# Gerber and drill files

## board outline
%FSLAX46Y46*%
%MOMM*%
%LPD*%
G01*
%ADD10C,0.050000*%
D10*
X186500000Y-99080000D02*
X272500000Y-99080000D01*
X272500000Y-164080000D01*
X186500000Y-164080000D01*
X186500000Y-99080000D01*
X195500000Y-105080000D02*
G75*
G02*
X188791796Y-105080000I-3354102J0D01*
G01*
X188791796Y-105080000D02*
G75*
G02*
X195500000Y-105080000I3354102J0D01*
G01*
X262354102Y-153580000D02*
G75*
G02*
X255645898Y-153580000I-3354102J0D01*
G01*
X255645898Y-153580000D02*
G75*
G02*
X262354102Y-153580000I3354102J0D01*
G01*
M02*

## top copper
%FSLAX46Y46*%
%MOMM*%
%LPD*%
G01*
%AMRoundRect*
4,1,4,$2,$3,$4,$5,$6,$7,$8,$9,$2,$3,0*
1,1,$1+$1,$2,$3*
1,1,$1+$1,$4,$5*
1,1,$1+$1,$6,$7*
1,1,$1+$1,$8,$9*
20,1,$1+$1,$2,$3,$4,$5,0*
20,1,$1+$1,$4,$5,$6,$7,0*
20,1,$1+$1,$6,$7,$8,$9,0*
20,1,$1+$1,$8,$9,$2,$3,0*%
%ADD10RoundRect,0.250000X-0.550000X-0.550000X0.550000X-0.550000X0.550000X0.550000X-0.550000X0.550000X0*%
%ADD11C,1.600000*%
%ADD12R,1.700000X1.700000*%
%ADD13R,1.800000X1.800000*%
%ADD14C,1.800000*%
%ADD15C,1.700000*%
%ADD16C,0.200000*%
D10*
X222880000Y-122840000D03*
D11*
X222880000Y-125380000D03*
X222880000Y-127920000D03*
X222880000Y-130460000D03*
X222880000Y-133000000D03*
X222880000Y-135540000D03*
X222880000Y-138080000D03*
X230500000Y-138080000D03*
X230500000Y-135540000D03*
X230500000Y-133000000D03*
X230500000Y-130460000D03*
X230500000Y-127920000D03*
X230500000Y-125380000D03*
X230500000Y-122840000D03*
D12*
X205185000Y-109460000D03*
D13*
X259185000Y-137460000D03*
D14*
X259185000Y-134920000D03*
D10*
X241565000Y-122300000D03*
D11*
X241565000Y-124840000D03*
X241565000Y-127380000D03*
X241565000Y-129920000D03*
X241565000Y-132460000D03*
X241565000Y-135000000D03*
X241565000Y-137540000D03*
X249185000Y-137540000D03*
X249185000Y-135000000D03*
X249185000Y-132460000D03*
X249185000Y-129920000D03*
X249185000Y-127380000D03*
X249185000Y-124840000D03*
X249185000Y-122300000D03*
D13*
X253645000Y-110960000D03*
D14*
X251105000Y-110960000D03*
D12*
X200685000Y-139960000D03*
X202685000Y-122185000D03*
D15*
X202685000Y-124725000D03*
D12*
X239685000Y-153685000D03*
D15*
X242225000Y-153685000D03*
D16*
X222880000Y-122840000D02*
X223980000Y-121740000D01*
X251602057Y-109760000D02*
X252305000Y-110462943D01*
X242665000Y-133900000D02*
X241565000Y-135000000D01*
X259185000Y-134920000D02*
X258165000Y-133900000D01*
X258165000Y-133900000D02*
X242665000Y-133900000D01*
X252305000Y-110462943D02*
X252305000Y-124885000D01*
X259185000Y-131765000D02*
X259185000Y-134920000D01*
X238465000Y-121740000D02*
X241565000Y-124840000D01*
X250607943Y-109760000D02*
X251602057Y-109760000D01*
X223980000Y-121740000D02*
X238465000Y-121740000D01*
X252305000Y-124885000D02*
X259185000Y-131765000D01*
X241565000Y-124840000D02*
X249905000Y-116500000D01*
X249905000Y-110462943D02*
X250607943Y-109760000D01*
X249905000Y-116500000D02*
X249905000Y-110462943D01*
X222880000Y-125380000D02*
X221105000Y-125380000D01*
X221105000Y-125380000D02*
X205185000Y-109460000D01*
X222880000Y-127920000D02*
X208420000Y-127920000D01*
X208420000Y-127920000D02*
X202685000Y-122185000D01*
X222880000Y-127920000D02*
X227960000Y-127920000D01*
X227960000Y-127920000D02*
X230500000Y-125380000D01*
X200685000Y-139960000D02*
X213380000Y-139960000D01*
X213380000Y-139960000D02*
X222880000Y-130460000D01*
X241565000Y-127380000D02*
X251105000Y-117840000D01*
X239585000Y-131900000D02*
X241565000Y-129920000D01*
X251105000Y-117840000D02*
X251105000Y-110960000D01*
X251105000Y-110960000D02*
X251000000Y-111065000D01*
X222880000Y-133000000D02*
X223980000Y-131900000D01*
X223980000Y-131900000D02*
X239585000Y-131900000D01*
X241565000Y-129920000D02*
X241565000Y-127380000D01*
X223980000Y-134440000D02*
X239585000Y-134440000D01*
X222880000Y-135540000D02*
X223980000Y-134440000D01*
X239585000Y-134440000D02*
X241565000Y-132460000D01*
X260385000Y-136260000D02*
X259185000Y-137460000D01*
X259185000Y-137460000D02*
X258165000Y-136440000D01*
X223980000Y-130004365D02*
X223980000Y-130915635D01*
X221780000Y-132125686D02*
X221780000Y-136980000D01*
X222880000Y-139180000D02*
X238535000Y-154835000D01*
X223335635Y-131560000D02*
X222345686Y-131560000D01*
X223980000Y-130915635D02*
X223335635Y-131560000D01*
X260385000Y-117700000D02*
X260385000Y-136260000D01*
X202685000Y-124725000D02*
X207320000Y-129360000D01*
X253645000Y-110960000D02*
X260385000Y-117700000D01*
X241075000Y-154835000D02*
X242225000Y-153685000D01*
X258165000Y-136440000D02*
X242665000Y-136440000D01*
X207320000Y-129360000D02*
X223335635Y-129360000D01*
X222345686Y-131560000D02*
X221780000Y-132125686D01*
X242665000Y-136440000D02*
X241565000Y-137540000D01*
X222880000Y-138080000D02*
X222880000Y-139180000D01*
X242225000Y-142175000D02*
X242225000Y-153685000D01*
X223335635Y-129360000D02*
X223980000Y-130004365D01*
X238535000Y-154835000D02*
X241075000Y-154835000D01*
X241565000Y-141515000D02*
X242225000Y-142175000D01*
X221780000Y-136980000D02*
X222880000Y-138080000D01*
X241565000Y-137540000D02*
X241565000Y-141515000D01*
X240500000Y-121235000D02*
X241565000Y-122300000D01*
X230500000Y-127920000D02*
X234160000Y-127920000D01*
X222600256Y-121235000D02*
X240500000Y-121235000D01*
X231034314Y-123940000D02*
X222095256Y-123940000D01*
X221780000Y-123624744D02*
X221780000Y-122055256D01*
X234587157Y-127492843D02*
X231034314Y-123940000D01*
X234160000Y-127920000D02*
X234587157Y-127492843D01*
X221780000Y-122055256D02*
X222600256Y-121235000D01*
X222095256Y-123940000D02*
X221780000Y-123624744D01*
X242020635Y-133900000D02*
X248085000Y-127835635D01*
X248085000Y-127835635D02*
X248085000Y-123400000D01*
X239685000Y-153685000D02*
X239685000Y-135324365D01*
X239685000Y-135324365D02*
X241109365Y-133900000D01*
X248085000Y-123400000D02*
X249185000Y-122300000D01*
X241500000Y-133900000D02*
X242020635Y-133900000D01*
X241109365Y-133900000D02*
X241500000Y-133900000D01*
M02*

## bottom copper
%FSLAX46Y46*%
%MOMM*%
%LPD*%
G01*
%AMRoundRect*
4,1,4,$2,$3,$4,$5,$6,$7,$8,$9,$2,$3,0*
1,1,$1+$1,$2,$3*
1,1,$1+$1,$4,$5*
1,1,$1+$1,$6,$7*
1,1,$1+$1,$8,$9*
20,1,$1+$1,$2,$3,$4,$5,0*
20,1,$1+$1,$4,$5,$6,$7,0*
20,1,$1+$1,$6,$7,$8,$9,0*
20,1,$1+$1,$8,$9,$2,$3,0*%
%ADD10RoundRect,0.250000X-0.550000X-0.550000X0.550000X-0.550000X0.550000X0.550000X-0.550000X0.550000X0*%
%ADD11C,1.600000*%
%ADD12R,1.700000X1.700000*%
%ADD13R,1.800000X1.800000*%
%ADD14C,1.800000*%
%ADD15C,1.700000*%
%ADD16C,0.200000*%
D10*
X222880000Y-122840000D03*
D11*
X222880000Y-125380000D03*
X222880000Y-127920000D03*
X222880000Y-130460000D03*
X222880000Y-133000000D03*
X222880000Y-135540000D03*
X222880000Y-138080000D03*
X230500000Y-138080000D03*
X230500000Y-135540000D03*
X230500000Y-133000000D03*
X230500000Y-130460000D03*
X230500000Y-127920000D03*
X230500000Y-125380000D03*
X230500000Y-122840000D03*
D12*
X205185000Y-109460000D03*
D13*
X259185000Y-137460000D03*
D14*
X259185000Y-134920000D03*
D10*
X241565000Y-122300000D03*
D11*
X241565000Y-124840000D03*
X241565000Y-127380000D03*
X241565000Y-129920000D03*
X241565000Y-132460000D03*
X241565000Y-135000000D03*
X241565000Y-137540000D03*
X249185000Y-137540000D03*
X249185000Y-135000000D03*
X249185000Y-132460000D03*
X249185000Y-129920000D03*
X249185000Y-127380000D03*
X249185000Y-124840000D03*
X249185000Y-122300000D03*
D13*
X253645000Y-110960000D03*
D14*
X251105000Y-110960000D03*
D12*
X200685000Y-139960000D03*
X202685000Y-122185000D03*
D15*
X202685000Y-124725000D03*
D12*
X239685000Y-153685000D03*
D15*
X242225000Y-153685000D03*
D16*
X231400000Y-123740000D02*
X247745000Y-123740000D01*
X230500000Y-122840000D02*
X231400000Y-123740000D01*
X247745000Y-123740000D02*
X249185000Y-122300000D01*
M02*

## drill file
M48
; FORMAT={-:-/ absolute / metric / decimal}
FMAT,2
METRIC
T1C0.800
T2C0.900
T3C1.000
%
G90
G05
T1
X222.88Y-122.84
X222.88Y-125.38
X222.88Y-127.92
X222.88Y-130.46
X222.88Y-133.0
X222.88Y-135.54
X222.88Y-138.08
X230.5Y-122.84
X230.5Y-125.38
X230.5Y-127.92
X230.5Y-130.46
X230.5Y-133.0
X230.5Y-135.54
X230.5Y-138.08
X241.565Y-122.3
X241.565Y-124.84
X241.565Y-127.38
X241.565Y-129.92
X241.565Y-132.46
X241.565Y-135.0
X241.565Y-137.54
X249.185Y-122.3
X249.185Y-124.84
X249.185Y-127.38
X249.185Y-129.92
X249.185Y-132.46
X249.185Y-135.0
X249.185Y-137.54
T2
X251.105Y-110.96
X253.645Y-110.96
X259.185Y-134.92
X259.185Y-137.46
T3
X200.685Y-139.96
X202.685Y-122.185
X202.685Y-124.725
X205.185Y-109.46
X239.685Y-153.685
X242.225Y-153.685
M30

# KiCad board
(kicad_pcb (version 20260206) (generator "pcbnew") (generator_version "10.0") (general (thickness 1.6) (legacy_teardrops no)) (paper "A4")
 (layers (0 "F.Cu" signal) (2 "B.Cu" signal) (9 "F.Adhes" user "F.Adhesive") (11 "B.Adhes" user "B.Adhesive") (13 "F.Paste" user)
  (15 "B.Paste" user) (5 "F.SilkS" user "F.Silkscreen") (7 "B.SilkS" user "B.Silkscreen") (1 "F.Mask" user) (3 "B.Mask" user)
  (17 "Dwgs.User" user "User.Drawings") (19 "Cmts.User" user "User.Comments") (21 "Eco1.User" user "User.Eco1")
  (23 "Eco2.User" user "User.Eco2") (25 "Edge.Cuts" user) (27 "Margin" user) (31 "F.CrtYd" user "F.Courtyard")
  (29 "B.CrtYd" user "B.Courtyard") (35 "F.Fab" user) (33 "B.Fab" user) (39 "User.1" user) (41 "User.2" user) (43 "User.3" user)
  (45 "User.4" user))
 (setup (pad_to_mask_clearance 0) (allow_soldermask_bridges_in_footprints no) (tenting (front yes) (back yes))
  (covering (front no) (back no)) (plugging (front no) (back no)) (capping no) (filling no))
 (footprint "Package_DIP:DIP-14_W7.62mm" (layer "F.Cu") (at 222.88 122.84)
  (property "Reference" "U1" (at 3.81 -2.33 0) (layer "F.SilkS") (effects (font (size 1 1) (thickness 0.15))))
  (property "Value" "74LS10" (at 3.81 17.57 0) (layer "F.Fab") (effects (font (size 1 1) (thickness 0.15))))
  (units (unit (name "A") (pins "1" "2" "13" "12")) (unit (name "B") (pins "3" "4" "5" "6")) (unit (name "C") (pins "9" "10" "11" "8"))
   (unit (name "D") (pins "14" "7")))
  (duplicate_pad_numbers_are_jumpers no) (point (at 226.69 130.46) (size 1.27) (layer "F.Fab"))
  (pad "1" thru_hole roundrect (at 0 0) (size 1.6 1.6) (drill 0.8) (layers "*.Cu" "*.Mask") (remove_unused_layers no)
   (roundrect_rratio 0.15625) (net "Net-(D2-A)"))
  (pad "2" thru_hole circle (at 0 2.54) (size 1.6 1.6) (drill 0.8) (layers "*.Cu" "*.Mask") (remove_unused_layers no) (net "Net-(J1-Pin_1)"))
  (pad "3" thru_hole circle (at 0 5.08) (size 1.6 1.6) (drill 0.8) (layers "*.Cu" "*.Mask") (remove_unused_layers no) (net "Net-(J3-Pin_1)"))
  (pad "4" thru_hole circle (at 0 7.62) (size 1.6 1.6) (drill 0.8) (layers "*.Cu" "*.Mask") (remove_unused_layers no) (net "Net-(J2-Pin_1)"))
  (pad "5" thru_hole circle (at 0 10.16) (size 1.6 1.6) (drill 0.8) (layers "*.Cu" "*.Mask") (remove_unused_layers no) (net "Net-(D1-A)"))
  (pad "6" thru_hole circle (at 0 12.7) (size 1.6 1.6) (drill 0.8) (layers "*.Cu" "*.Mask") (remove_unused_layers no) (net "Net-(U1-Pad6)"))
  (pad "7" thru_hole circle (at 0 15.24) (size 1.6 1.6) (drill 0.8) (layers "*.Cu" "*.Mask") (remove_unused_layers no) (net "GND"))
  (pad "8" thru_hole circle (at 7.62 15.24) (size 1.6 1.6) (drill 0.8) (layers "*.Cu" "*.Mask") (remove_unused_layers no))
  (pad "9" thru_hole circle (at 7.62 12.7) (size 1.6 1.6) (drill 0.8) (layers "*.Cu" "*.Mask") (remove_unused_layers no))
  (pad "10" thru_hole circle (at 7.62 10.16) (size 1.6 1.6) (drill 0.8) (layers "*.Cu" "*.Mask") (remove_unused_layers no))
  (pad "11" thru_hole circle (at 7.62 7.62) (size 1.6 1.6) (drill 0.8) (layers "*.Cu" "*.Mask") (remove_unused_layers no))
  (pad "12" thru_hole circle (at 7.62 5.08) (size 1.6 1.6) (drill 0.8) (layers "*.Cu" "*.Mask") (remove_unused_layers no)
   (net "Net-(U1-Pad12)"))
  (pad "13" thru_hole circle (at 7.62 2.54) (size 1.6 1.6) (drill 0.8) (layers "*.Cu" "*.Mask") (remove_unused_layers no)
   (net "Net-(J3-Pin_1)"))
  (pad "14" thru_hole circle (at 7.62 0) (size 1.6 1.6) (drill 0.8) (layers "*.Cu" "*.Mask") (remove_unused_layers no) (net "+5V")))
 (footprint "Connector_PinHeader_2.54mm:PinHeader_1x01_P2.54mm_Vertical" (layer "F.Cu") (at 205.185 109.46)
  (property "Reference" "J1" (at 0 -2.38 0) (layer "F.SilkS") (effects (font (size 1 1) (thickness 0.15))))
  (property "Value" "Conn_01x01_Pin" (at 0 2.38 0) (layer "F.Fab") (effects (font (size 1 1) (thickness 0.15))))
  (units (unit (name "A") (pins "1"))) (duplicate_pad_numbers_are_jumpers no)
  (pad "1" thru_hole rect (at 0 0) (size 1.7 1.7) (drill 1) (layers "*.Cu" "*.Mask") (remove_unused_layers no) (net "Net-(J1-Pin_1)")))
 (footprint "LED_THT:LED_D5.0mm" (layer "F.Cu") (at 259.185 137.46 90)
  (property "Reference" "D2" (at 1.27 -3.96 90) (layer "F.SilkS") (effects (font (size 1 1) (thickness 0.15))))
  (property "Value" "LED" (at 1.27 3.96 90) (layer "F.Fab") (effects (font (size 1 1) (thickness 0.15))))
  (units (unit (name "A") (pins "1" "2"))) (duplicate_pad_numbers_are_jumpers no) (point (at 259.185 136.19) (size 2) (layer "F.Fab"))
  (pad "1" thru_hole rect (at 0 0 90) (size 1.8 1.8) (drill 0.9) (layers "*.Cu" "*.Mask") (remove_unused_layers no) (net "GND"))
  (pad "2" thru_hole circle (at 2.54 0 90) (size 1.8 1.8) (drill 0.9) (layers "*.Cu" "*.Mask") (remove_unused_layers no) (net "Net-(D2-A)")))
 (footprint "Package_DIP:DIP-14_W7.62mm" (layer "F.Cu") (at 241.565 122.3)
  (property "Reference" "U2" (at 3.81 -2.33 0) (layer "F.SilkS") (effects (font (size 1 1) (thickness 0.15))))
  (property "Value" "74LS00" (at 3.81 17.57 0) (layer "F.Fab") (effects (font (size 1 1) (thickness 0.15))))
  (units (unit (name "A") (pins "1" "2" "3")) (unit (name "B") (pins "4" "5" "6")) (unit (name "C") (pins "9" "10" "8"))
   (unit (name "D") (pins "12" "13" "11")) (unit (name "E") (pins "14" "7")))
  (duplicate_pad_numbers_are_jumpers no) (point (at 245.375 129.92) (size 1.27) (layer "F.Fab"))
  (pad "1" thru_hole roundrect (at 0 0) (size 1.6 1.6) (drill 0.8) (layers "*.Cu" "*.Mask") (remove_unused_layers no)
   (roundrect_rratio 0.15625) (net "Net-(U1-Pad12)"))
  (pad "2" thru_hole circle (at 0 2.54) (size 1.6 1.6) (drill 0.8) (layers "*.Cu" "*.Mask") (remove_unused_layers no) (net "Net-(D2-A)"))
  (pad "3" thru_hole circle (at 0 5.08) (size 1.6 1.6) (drill 0.8) (layers "*.Cu" "*.Mask") (remove_unused_layers no) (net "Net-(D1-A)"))
  (pad "4" thru_hole circle (at 0 7.62) (size 1.6 1.6) (drill 0.8) (layers "*.Cu" "*.Mask") (remove_unused_layers no) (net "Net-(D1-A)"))
  (pad "5" thru_hole circle (at 0 10.16) (size 1.6 1.6) (drill 0.8) (layers "*.Cu" "*.Mask") (remove_unused_layers no) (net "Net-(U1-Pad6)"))
  (pad "6" thru_hole circle (at 0 12.7) (size 1.6 1.6) (drill 0.8) (layers "*.Cu" "*.Mask") (remove_unused_layers no) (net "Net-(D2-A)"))
  (pad "7" thru_hole circle (at 0 15.24) (size 1.6 1.6) (drill 0.8) (layers "*.Cu" "*.Mask") (remove_unused_layers no) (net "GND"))
  (pad "8" thru_hole circle (at 7.62 15.24) (size 1.6 1.6) (drill 0.8) (layers "*.Cu" "*.Mask") (remove_unused_layers no))
  (pad "9" thru_hole circle (at 7.62 12.7) (size 1.6 1.6) (drill 0.8) (layers "*.Cu" "*.Mask") (remove_unused_layers no))
  (pad "10" thru_hole circle (at 7.62 10.16) (size 1.6 1.6) (drill 0.8) (layers "*.Cu" "*.Mask") (remove_unused_layers no))
  (pad "11" thru_hole circle (at 7.62 7.62) (size 1.6 1.6) (drill 0.8) (layers "*.Cu" "*.Mask") (remove_unused_layers no))
  (pad "12" thru_hole circle (at 7.62 5.08) (size 1.6 1.6) (drill 0.8) (layers "*.Cu" "*.Mask") (remove_unused_layers no))
  (pad "13" thru_hole circle (at 7.62 2.54) (size 1.6 1.6) (drill 0.8) (layers "*.Cu" "*.Mask") (remove_unused_layers no))
  (pad "14" thru_hole circle (at 7.62 0) (size 1.6 1.6) (drill 0.8) (layers "*.Cu" "*.Mask") (remove_unused_layers no) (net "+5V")))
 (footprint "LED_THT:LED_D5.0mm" (layer "F.Cu") (at 253.645 110.96 180)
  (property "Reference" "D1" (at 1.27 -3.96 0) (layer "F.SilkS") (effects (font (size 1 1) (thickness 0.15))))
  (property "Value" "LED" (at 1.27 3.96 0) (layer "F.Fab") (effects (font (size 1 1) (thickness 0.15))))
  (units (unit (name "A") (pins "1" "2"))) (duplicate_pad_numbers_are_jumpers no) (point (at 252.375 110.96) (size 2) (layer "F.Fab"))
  (pad "1" thru_hole rect (at 0 0 180) (size 1.8 1.8) (drill 0.9) (layers "*.Cu" "*.Mask") (remove_unused_layers no) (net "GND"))
  (pad "2" thru_hole circle (at 2.54 0 180) (size 1.8 1.8) (drill 0.9) (layers "*.Cu" "*.Mask") (remove_unused_layers no) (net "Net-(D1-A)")))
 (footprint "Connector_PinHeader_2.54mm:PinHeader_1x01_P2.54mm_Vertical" (layer "F.Cu") (at 200.685 139.96)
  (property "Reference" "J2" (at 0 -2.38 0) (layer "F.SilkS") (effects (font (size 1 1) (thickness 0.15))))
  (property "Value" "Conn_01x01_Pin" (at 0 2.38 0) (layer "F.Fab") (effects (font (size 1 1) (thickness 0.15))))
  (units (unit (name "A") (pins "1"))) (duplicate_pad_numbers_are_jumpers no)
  (pad "1" thru_hole rect (at 0 0) (size 1.7 1.7) (drill 1) (layers "*.Cu" "*.Mask") (remove_unused_layers no) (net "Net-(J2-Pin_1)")))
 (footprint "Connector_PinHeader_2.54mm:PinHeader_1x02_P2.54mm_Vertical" (layer "F.Cu") (at 202.685 122.185)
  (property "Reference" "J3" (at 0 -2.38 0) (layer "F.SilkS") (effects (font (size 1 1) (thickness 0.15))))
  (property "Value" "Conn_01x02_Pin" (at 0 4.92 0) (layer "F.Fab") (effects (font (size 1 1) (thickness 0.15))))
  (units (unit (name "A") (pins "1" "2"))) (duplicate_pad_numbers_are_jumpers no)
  (pad "1" thru_hole rect (at 0 0) (size 1.7 1.7) (drill 1) (layers "*.Cu" "*.Mask") (remove_unused_layers no) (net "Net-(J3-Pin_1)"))
  (pad "2" thru_hole circle (at 0 2.54) (size 1.7 1.7) (drill 1) (layers "*.Cu" "*.Mask") (remove_unused_layers no) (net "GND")))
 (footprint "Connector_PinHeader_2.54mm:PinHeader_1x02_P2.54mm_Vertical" (layer "F.Cu") (at 239.685 153.685 90)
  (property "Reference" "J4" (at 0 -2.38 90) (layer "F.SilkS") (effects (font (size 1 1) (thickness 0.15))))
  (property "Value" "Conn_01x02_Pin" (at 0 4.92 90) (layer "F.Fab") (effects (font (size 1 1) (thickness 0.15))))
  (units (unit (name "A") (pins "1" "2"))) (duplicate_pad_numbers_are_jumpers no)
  (pad "1" thru_hole rect (at 0 0 90) (size 1.7 1.7) (drill 1) (layers "*.Cu" "*.Mask") (remove_unused_layers no) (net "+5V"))
  (pad "2" thru_hole circle (at 0 2.54 90) (size 1.7 1.7) (drill 1) (layers "*.Cu" "*.Mask") (remove_unused_layers no) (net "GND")))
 (gr_rect (start 186.5 99.08) (end 272.5 164.08) (stroke (width 0.05) (type default)) (fill no) (layer "Edge.Cuts"))
 (gr_circle (center 192.145898 105.08) (end 193.645898 108.08) (stroke (width 0.05) (type default)) (fill no) (layer "Edge.Cuts"))
 (gr_circle (center 259 153.58) (end 260.5 156.58) (stroke (width 0.05) (type default)) (fill no) (layer "Edge.Cuts"))
 (segment (start 222.88 122.84) (end 223.98 121.74) (width 0.2) (layer "F.Cu") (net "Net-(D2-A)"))
 (segment (start 251.602057 109.76) (end 252.305 110.462943) (width 0.2) (layer "F.Cu") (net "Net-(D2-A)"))
 (segment (start 242.665 133.9) (end 241.565 135) (width 0.2) (layer "F.Cu") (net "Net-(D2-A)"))
 (segment (start 259.185 134.92) (end 258.165 133.9) (width 0.2) (layer "F.Cu") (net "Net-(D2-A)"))
 (segment (start 258.165 133.9) (end 242.665 133.9) (width 0.2) (layer "F.Cu") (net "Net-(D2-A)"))
 (segment (start 252.305 110.462943) (end 252.305 124.885) (width 0.2) (layer "F.Cu") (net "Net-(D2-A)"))
 (segment (start 259.185 131.765) (end 259.185 134.92) (width 0.2) (layer "F.Cu") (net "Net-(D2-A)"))
 (segment (start 238.465 121.74) (end 241.565 124.84) (width 0.2) (layer "F.Cu") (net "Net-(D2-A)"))
 (segment (start 250.607943 109.76) (end 251.602057 109.76) (width 0.2) (layer "F.Cu") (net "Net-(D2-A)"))
 (segment (start 223.98 121.74) (end 238.465 121.74) (width 0.2) (layer "F.Cu") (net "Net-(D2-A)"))
 (segment (start 252.305 124.885) (end 259.185 131.765) (width 0.2) (layer "F.Cu") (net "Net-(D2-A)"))
 (segment (start 241.565 124.84) (end 249.905 116.5) (width 0.2) (layer "F.Cu") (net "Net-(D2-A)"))
 (segment (start 249.905 110.462943) (end 250.607943 109.76) (width 0.2) (layer "F.Cu") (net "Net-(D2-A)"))
 (segment (start 249.905 116.5) (end 249.905 110.462943) (width 0.2) (layer "F.Cu") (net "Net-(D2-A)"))
 (segment (start 222.88 125.38) (end 221.105 125.38) (width 0.2) (layer "F.Cu") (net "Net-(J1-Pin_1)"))
 (segment (start 221.105 125.38) (end 205.185 109.46) (width 0.2) (layer "F.Cu") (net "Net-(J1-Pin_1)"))
 (segment (start 222.88 127.92) (end 208.42 127.92) (width 0.2) (layer "F.Cu") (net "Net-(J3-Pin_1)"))
 (segment (start 208.42 127.92) (end 202.685 122.185) (width 0.2) (layer "F.Cu") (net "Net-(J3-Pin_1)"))
 (segment (start 222.88 127.92) (end 227.96 127.92) (width 0.2) (layer "F.Cu") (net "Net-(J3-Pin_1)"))
 (segment (start 227.96 127.92) (end 230.5 125.38) (width 0.2) (layer "F.Cu") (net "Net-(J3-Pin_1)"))
 (segment (start 200.685 139.96) (end 213.38 139.96) (width 0.2) (layer "F.Cu") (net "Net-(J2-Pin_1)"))
 (segment (start 213.38 139.96) (end 222.88 130.46) (width 0.2) (layer "F.Cu") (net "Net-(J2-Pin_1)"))
 (segment (start 241.565 127.38) (end 251.105 117.84) (width 0.2) (layer "F.Cu") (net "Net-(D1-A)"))
 (segment (start 239.585 131.9) (end 241.565 129.92) (width 0.2) (layer "F.Cu") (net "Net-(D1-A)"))
 (segment (start 251.105 117.84) (end 251.105 110.96) (width 0.2) (layer "F.Cu") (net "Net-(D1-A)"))
 (segment (start 251.105 110.96) (end 251 111.065) (width 0.2) (layer "F.Cu") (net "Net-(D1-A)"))
 (segment (start 222.88 133) (end 223.98 131.9) (width 0.2) (layer "F.Cu") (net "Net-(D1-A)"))
 (segment (start 223.98 131.9) (end 239.585 131.9) (width 0.2) (layer "F.Cu") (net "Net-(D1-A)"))
 (segment (start 241.565 129.92) (end 241.565 127.38) (width 0.2) (layer "F.Cu") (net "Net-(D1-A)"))
 (segment (start 223.98 134.44) (end 239.585 134.44) (width 0.2) (layer "F.Cu") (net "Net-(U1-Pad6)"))
 (segment (start 222.88 135.54) (end 223.98 134.44) (width 0.2) (layer "F.Cu") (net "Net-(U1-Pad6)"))
 (segment (start 239.585 134.44) (end 241.565 132.46) (width 0.2) (layer "F.Cu") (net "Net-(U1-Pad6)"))
 (segment (start 260.385 136.26) (end 259.185 137.46) (width 0.2) (layer "F.Cu") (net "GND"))
 (segment (start 259.185 137.46) (end 258.165 136.44) (width 0.2) (layer "F.Cu") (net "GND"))
 (segment (start 223.98 130.004365) (end 223.98 130.915635) (width 0.2) (layer "F.Cu") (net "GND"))
 (segment (start 221.78 132.125686) (end 221.78 136.98) (width 0.2) (layer "F.Cu") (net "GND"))
 (segment (start 222.88 139.18) (end 238.535 154.835) (width 0.2) (layer "F.Cu") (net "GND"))
 (segment (start 223.335635 131.56) (end 222.345686 131.56) (width 0.2) (layer "F.Cu") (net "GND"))
 (segment (start 223.98 130.915635) (end 223.335635 131.56) (width 0.2) (layer "F.Cu") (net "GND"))
 (segment (start 260.385 117.7) (end 260.385 136.26) (width 0.2) (layer "F.Cu") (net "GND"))
 (segment (start 202.685 124.725) (end 207.32 129.36) (width 0.2) (layer "F.Cu") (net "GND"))
 (segment (start 253.645 110.96) (end 260.385 117.7) (width 0.2) (layer "F.Cu") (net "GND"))
 (segment (start 241.075 154.835) (end 242.225 153.685) (width 0.2) (layer "F.Cu") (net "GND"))
 (segment (start 258.165 136.44) (end 242.665 136.44) (width 0.2) (layer "F.Cu") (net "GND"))
 (segment (start 207.32 129.36) (end 223.335635 129.36) (width 0.2) (layer "F.Cu") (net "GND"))
 (segment (start 222.345686 131.56) (end 221.78 132.125686) (width 0.2) (layer "F.Cu") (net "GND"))
 (segment (start 242.665 136.44) (end 241.565 137.54) (width 0.2) (layer "F.Cu") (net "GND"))
 (segment (start 222.88 138.08) (end 222.88 139.18) (width 0.2) (layer "F.Cu") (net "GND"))
 (segment (start 242.225 142.175) (end 242.225 153.685) (width 0.2) (layer "F.Cu") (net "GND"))
 (segment (start 223.335635 129.36) (end 223.98 130.004365) (width 0.2) (layer "F.Cu") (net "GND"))
 (segment (start 238.535 154.835) (end 241.075 154.835) (width 0.2) (layer "F.Cu") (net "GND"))
 (segment (start 241.565 141.515) (end 242.225 142.175) (width 0.2) (layer "F.Cu") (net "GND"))
 (segment (start 221.78 136.98) (end 222.88 138.08) (width 0.2) (layer "F.Cu") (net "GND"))
 (segment (start 241.565 137.54) (end 241.565 141.515) (width 0.2) (layer "F.Cu") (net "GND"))
 (segment (start 240.5 121.235) (end 241.565 122.3) (width 0.2) (layer "F.Cu") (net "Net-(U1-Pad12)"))
 (segment (start 230.5 127.92) (end 234.16 127.92) (width 0.2) (layer "F.Cu") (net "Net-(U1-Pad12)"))
 (segment (start 222.600256 121.235) (end 240.5 121.235) (width 0.2) (layer "F.Cu") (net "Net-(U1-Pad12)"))
 (segment (start 231.034314 123.94) (end 222.095256 123.94) (width 0.2) (layer "F.Cu") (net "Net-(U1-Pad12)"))
 (segment (start 221.78 123.624744) (end 221.78 122.055256) (width 0.2) (layer "F.Cu") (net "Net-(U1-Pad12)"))
 (segment (start 234.587157 127.492843) (end 231.034314 123.94) (width 0.2) (layer "F.Cu") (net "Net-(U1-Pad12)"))
 (segment (start 234.16 127.92) (end 234.587157 127.492843) (width 0.2) (layer "F.Cu") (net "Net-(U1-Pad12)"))
 (segment (start 221.78 122.055256) (end 222.600256 121.235) (width 0.2) (layer "F.Cu") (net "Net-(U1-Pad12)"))
 (segment (start 222.095256 123.94) (end 221.78 123.624744) (width 0.2) (layer "F.Cu") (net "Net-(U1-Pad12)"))
 (segment (start 242.020635 133.9) (end 248.085 127.835635) (width 0.2) (layer "F.Cu") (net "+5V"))
 (segment (start 248.085 127.835635) (end 248.085 123.4) (width 0.2) (layer "F.Cu") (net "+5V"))
 (segment (start 239.685 153.685) (end 239.685 135.324365) (width 0.2) (layer "F.Cu") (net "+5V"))
 (segment (start 239.685 135.324365) (end 241.109365 133.9) (width 0.2) (layer "F.Cu") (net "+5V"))
 (segment (start 248.085 123.4) (end 249.185 122.3) (width 0.2) (layer "F.Cu") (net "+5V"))
 (segment (start 241.5 133.9) (end 242.020635 133.9) (width 0.2) (layer "F.Cu") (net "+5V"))
 (segment (start 241.109365 133.9) (end 241.5 133.9) (width 0.2) (layer "F.Cu") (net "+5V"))
 (segment (start 231.4 123.74) (end 247.745 123.74) (width 0.2) (layer "B.Cu") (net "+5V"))
 (segment (start 230.5 122.84) (end 231.4 123.74) (width 0.2) (layer "B.Cu") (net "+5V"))
 (segment (start 247.745 123.74) (end 249.185 122.3) (width 0.2) (layer "B.Cu") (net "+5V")))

